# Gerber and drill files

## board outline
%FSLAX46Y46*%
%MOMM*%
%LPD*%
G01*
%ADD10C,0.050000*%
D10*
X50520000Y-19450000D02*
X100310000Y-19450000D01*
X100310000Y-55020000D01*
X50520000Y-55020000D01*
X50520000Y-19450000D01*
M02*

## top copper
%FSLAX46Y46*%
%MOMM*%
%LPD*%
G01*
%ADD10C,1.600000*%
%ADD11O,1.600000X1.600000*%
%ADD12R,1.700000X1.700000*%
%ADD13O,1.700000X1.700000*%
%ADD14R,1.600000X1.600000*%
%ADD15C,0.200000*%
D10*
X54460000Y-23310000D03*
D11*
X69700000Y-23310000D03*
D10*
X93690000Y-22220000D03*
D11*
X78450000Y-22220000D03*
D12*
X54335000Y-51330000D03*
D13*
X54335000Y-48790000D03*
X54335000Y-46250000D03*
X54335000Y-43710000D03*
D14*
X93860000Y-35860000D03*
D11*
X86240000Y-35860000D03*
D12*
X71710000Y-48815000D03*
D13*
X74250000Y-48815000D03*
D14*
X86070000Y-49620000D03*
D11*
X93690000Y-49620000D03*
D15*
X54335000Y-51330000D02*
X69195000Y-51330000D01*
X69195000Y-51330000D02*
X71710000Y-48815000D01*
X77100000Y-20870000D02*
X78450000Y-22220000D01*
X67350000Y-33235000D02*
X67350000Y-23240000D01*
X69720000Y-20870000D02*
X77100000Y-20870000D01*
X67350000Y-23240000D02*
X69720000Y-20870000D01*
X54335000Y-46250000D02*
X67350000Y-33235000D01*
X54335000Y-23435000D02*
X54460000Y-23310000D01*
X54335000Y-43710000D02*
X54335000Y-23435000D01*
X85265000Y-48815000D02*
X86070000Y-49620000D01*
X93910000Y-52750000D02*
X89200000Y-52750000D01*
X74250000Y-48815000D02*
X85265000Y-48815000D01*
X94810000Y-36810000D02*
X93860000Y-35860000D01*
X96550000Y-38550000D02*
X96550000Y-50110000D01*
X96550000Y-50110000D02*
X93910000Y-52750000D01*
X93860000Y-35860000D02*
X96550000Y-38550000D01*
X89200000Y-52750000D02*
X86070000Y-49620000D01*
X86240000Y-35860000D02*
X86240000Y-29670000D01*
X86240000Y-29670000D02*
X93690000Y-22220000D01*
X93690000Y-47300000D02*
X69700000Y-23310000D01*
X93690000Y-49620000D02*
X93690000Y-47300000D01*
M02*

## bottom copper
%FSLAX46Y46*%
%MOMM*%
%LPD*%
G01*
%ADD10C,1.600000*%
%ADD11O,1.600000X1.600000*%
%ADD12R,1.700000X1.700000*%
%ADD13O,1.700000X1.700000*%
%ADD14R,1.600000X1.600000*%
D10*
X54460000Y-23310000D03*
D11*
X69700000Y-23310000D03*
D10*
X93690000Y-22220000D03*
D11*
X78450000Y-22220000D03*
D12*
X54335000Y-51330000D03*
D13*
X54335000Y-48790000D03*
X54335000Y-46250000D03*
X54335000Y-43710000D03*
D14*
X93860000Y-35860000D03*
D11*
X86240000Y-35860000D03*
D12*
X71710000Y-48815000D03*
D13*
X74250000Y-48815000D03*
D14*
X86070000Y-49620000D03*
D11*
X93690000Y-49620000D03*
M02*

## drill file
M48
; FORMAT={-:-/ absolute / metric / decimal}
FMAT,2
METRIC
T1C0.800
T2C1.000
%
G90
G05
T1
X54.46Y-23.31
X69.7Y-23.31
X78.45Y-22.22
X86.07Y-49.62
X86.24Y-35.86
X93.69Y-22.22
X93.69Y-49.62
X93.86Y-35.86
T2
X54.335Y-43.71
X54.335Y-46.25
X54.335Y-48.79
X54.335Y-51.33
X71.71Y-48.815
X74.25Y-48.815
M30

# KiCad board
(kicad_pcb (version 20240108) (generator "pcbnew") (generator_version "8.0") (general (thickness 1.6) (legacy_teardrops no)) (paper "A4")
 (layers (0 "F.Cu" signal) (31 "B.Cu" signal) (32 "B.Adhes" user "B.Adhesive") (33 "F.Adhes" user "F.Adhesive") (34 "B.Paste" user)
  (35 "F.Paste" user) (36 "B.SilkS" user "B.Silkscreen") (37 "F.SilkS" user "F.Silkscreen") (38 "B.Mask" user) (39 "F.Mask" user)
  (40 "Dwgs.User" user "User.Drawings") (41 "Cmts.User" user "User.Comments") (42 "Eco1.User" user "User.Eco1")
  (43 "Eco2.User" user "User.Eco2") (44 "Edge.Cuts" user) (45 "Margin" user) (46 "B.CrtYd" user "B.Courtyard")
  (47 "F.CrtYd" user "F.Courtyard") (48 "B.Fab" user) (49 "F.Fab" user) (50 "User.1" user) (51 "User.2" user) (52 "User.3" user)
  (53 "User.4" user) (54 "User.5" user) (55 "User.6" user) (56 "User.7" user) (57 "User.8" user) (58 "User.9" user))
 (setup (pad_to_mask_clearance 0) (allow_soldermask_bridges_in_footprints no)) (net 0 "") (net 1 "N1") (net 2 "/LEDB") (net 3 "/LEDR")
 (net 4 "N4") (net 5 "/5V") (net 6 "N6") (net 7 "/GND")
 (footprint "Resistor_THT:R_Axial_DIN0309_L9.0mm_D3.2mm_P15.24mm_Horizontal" (layer "F.Cu") (at 54.46 23.31)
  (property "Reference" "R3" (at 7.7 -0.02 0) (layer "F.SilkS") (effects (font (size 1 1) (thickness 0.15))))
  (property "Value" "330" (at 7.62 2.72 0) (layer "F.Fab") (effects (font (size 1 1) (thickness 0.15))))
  (pad "1" thru_hole circle (at 0 0) (size 1.6 1.6) (drill 0.8) (layers "*.Cu" "*.Mask") (remove_unused_layers no) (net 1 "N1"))
  (pad "2" thru_hole oval (at 15.24 0) (size 1.6 1.6) (drill 0.8) (layers "*.Cu" "*.Mask") (remove_unused_layers no) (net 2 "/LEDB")))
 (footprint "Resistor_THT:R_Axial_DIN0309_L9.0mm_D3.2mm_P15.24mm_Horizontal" (layer "F.Cu") (at 93.69 22.22 180)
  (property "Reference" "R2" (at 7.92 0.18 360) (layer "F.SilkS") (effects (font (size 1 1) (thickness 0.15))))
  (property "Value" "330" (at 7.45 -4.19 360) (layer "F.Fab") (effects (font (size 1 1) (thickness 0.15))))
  (pad "1" thru_hole circle (at 0 0 180) (size 1.6 1.6) (drill 0.8) (layers "*.Cu" "*.Mask") (remove_unused_layers no) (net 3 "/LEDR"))
  (pad "2" thru_hole oval (at 15.24 0 180) (size 1.6 1.6) (drill 0.8) (layers "*.Cu" "*.Mask") (remove_unused_layers no) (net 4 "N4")))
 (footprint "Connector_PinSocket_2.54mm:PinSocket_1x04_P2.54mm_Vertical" (layer "F.Cu") (at 54.335 51.33 180)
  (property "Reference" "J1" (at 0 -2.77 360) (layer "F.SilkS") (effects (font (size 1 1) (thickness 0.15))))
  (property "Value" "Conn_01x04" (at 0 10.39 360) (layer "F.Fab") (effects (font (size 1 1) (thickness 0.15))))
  (pad "1" thru_hole rect (at 0 0 180) (size 1.7 1.7) (drill 1) (layers "*.Cu" "*.Mask") (remove_unused_layers no) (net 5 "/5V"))
  (pad "2" thru_hole oval (at 0 2.54 180) (size 1.7 1.7) (drill 1) (layers "*.Cu" "*.Mask") (remove_unused_layers no) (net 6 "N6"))
  (pad "3" thru_hole oval (at 0 5.08 180) (size 1.7 1.7) (drill 1) (layers "*.Cu" "*.Mask") (remove_unused_layers no) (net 4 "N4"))
  (pad "4" thru_hole oval (at 0 7.62 180) (size 1.7 1.7) (drill 1) (layers "*.Cu" "*.Mask") (remove_unused_layers no) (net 1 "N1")))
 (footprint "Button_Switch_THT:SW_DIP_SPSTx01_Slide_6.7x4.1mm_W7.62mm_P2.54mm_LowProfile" (layer "F.Cu") (at 93.86 35.86 180)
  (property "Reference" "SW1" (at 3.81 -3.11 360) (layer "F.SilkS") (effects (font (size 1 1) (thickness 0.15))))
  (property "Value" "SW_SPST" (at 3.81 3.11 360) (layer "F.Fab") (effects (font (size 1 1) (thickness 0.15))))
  (pad "1" thru_hole rect (at 0 0 180) (size 1.6 1.6) (drill 0.8) (layers "*.Cu" "*.Mask") (remove_unused_layers no) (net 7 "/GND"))
  (pad "2" thru_hole oval (at 7.62 0 180) (size 1.6 1.6) (drill 0.8) (layers "*.Cu" "*.Mask") (remove_unused_layers no) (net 3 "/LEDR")))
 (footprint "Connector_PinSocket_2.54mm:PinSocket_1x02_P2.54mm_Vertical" (layer "F.Cu") (at 71.71 48.815 90)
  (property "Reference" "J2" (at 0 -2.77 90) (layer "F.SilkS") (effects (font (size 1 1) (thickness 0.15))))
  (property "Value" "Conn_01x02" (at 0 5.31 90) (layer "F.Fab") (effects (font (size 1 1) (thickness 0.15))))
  (pad "1" thru_hole rect (at 0 0 90) (size 1.7 1.7) (drill 1) (layers "*.Cu" "*.Mask") (remove_unused_layers no) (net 5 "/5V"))
  (pad "2" thru_hole oval (at 0 2.54 90) (size 1.7 1.7) (drill 1) (layers "*.Cu" "*.Mask") (remove_unused_layers no) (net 7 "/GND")))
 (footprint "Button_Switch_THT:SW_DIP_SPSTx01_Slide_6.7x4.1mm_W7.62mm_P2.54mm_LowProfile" (layer "F.Cu") (at 86.07 49.62)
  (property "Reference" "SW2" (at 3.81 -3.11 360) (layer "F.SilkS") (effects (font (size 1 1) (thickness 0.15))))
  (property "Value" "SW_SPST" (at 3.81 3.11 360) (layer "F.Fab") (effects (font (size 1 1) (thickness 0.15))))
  (pad "1" thru_hole rect (at 0 0) (size 1.6 1.6) (drill 0.8) (layers "*.Cu" "*.Mask") (remove_unused_layers no) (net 7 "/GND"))
  (pad "2" thru_hole oval (at 7.62 0) (size 1.6 1.6) (drill 0.8) (layers "*.Cu" "*.Mask") (remove_unused_layers no) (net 2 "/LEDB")))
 (gr_rect (start 50.52 19.45) (end 100.31 55.02) (stroke (width 0.05) (type default)) (fill none) (layer "Edge.Cuts"))
 (segment (start 54.335 51.33) (end 69.195 51.33) (width 0.2) (layer "F.Cu") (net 5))
 (segment (start 69.195 51.33) (end 71.71 48.815) (width 0.2) (layer "F.Cu") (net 5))
 (segment (start 77.1 20.87) (end 78.45 22.22) (width 0.2) (layer "F.Cu") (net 4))
 (segment (start 67.35 33.235) (end 67.35 23.24) (width 0.2) (layer "F.Cu") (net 4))
 (segment (start 69.72 20.87) (end 77.1 20.87) (width 0.2) (layer "F.Cu") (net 4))
 (segment (start 67.35 23.24) (end 69.72 20.87) (width 0.2) (layer "F.Cu") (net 4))
 (segment (start 54.335 46.25) (end 67.35 33.235) (width 0.2) (layer "F.Cu") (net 4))
 (segment (start 54.335 23.435) (end 54.46 23.31) (width 0.2) (layer "F.Cu") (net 1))
 (segment (start 54.335 43.71) (end 54.335 23.435) (width 0.2) (layer "F.Cu") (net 1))
 (segment (start 85.265 48.815) (end 86.07 49.62) (width 0.2) (layer "F.Cu") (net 7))
 (segment (start 93.91 52.75) (end 89.2 52.75) (width 0.2) (layer "F.Cu") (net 7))
 (segment (start 74.25 48.815) (end 85.265 48.815) (width 0.2) (layer "F.Cu") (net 7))
 (segment (start 94.81 36.81) (end 93.86 35.86) (width 0.2) (layer "F.Cu") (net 7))
 (segment (start 96.55 38.55) (end 96.55 50.11) (width 0.2) (layer "F.Cu") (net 7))
 (segment (start 96.55 50.11) (end 93.91 52.75) (width 0.2) (layer "F.Cu") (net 7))
 (segment (start 93.86 35.86) (end 96.55 38.55) (width 0.2) (layer "F.Cu") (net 7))
 (segment (start 89.2 52.75) (end 86.07 49.62) (width 0.2) (layer "F.Cu") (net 7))
 (segment (start 86.24 35.86) (end 86.24 29.67) (width 0.2) (layer "F.Cu") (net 3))
 (segment (start 86.24 29.67) (end 93.69 22.22) (width 0.2) (layer "F.Cu") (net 3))
 (segment (start 93.69 47.3) (end 69.7 23.31) (width 0.2) (layer "F.Cu") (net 2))
 (segment (start 93.69 49.62) (end 93.69 47.3) (width 0.2) (layer "F.Cu") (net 2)))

